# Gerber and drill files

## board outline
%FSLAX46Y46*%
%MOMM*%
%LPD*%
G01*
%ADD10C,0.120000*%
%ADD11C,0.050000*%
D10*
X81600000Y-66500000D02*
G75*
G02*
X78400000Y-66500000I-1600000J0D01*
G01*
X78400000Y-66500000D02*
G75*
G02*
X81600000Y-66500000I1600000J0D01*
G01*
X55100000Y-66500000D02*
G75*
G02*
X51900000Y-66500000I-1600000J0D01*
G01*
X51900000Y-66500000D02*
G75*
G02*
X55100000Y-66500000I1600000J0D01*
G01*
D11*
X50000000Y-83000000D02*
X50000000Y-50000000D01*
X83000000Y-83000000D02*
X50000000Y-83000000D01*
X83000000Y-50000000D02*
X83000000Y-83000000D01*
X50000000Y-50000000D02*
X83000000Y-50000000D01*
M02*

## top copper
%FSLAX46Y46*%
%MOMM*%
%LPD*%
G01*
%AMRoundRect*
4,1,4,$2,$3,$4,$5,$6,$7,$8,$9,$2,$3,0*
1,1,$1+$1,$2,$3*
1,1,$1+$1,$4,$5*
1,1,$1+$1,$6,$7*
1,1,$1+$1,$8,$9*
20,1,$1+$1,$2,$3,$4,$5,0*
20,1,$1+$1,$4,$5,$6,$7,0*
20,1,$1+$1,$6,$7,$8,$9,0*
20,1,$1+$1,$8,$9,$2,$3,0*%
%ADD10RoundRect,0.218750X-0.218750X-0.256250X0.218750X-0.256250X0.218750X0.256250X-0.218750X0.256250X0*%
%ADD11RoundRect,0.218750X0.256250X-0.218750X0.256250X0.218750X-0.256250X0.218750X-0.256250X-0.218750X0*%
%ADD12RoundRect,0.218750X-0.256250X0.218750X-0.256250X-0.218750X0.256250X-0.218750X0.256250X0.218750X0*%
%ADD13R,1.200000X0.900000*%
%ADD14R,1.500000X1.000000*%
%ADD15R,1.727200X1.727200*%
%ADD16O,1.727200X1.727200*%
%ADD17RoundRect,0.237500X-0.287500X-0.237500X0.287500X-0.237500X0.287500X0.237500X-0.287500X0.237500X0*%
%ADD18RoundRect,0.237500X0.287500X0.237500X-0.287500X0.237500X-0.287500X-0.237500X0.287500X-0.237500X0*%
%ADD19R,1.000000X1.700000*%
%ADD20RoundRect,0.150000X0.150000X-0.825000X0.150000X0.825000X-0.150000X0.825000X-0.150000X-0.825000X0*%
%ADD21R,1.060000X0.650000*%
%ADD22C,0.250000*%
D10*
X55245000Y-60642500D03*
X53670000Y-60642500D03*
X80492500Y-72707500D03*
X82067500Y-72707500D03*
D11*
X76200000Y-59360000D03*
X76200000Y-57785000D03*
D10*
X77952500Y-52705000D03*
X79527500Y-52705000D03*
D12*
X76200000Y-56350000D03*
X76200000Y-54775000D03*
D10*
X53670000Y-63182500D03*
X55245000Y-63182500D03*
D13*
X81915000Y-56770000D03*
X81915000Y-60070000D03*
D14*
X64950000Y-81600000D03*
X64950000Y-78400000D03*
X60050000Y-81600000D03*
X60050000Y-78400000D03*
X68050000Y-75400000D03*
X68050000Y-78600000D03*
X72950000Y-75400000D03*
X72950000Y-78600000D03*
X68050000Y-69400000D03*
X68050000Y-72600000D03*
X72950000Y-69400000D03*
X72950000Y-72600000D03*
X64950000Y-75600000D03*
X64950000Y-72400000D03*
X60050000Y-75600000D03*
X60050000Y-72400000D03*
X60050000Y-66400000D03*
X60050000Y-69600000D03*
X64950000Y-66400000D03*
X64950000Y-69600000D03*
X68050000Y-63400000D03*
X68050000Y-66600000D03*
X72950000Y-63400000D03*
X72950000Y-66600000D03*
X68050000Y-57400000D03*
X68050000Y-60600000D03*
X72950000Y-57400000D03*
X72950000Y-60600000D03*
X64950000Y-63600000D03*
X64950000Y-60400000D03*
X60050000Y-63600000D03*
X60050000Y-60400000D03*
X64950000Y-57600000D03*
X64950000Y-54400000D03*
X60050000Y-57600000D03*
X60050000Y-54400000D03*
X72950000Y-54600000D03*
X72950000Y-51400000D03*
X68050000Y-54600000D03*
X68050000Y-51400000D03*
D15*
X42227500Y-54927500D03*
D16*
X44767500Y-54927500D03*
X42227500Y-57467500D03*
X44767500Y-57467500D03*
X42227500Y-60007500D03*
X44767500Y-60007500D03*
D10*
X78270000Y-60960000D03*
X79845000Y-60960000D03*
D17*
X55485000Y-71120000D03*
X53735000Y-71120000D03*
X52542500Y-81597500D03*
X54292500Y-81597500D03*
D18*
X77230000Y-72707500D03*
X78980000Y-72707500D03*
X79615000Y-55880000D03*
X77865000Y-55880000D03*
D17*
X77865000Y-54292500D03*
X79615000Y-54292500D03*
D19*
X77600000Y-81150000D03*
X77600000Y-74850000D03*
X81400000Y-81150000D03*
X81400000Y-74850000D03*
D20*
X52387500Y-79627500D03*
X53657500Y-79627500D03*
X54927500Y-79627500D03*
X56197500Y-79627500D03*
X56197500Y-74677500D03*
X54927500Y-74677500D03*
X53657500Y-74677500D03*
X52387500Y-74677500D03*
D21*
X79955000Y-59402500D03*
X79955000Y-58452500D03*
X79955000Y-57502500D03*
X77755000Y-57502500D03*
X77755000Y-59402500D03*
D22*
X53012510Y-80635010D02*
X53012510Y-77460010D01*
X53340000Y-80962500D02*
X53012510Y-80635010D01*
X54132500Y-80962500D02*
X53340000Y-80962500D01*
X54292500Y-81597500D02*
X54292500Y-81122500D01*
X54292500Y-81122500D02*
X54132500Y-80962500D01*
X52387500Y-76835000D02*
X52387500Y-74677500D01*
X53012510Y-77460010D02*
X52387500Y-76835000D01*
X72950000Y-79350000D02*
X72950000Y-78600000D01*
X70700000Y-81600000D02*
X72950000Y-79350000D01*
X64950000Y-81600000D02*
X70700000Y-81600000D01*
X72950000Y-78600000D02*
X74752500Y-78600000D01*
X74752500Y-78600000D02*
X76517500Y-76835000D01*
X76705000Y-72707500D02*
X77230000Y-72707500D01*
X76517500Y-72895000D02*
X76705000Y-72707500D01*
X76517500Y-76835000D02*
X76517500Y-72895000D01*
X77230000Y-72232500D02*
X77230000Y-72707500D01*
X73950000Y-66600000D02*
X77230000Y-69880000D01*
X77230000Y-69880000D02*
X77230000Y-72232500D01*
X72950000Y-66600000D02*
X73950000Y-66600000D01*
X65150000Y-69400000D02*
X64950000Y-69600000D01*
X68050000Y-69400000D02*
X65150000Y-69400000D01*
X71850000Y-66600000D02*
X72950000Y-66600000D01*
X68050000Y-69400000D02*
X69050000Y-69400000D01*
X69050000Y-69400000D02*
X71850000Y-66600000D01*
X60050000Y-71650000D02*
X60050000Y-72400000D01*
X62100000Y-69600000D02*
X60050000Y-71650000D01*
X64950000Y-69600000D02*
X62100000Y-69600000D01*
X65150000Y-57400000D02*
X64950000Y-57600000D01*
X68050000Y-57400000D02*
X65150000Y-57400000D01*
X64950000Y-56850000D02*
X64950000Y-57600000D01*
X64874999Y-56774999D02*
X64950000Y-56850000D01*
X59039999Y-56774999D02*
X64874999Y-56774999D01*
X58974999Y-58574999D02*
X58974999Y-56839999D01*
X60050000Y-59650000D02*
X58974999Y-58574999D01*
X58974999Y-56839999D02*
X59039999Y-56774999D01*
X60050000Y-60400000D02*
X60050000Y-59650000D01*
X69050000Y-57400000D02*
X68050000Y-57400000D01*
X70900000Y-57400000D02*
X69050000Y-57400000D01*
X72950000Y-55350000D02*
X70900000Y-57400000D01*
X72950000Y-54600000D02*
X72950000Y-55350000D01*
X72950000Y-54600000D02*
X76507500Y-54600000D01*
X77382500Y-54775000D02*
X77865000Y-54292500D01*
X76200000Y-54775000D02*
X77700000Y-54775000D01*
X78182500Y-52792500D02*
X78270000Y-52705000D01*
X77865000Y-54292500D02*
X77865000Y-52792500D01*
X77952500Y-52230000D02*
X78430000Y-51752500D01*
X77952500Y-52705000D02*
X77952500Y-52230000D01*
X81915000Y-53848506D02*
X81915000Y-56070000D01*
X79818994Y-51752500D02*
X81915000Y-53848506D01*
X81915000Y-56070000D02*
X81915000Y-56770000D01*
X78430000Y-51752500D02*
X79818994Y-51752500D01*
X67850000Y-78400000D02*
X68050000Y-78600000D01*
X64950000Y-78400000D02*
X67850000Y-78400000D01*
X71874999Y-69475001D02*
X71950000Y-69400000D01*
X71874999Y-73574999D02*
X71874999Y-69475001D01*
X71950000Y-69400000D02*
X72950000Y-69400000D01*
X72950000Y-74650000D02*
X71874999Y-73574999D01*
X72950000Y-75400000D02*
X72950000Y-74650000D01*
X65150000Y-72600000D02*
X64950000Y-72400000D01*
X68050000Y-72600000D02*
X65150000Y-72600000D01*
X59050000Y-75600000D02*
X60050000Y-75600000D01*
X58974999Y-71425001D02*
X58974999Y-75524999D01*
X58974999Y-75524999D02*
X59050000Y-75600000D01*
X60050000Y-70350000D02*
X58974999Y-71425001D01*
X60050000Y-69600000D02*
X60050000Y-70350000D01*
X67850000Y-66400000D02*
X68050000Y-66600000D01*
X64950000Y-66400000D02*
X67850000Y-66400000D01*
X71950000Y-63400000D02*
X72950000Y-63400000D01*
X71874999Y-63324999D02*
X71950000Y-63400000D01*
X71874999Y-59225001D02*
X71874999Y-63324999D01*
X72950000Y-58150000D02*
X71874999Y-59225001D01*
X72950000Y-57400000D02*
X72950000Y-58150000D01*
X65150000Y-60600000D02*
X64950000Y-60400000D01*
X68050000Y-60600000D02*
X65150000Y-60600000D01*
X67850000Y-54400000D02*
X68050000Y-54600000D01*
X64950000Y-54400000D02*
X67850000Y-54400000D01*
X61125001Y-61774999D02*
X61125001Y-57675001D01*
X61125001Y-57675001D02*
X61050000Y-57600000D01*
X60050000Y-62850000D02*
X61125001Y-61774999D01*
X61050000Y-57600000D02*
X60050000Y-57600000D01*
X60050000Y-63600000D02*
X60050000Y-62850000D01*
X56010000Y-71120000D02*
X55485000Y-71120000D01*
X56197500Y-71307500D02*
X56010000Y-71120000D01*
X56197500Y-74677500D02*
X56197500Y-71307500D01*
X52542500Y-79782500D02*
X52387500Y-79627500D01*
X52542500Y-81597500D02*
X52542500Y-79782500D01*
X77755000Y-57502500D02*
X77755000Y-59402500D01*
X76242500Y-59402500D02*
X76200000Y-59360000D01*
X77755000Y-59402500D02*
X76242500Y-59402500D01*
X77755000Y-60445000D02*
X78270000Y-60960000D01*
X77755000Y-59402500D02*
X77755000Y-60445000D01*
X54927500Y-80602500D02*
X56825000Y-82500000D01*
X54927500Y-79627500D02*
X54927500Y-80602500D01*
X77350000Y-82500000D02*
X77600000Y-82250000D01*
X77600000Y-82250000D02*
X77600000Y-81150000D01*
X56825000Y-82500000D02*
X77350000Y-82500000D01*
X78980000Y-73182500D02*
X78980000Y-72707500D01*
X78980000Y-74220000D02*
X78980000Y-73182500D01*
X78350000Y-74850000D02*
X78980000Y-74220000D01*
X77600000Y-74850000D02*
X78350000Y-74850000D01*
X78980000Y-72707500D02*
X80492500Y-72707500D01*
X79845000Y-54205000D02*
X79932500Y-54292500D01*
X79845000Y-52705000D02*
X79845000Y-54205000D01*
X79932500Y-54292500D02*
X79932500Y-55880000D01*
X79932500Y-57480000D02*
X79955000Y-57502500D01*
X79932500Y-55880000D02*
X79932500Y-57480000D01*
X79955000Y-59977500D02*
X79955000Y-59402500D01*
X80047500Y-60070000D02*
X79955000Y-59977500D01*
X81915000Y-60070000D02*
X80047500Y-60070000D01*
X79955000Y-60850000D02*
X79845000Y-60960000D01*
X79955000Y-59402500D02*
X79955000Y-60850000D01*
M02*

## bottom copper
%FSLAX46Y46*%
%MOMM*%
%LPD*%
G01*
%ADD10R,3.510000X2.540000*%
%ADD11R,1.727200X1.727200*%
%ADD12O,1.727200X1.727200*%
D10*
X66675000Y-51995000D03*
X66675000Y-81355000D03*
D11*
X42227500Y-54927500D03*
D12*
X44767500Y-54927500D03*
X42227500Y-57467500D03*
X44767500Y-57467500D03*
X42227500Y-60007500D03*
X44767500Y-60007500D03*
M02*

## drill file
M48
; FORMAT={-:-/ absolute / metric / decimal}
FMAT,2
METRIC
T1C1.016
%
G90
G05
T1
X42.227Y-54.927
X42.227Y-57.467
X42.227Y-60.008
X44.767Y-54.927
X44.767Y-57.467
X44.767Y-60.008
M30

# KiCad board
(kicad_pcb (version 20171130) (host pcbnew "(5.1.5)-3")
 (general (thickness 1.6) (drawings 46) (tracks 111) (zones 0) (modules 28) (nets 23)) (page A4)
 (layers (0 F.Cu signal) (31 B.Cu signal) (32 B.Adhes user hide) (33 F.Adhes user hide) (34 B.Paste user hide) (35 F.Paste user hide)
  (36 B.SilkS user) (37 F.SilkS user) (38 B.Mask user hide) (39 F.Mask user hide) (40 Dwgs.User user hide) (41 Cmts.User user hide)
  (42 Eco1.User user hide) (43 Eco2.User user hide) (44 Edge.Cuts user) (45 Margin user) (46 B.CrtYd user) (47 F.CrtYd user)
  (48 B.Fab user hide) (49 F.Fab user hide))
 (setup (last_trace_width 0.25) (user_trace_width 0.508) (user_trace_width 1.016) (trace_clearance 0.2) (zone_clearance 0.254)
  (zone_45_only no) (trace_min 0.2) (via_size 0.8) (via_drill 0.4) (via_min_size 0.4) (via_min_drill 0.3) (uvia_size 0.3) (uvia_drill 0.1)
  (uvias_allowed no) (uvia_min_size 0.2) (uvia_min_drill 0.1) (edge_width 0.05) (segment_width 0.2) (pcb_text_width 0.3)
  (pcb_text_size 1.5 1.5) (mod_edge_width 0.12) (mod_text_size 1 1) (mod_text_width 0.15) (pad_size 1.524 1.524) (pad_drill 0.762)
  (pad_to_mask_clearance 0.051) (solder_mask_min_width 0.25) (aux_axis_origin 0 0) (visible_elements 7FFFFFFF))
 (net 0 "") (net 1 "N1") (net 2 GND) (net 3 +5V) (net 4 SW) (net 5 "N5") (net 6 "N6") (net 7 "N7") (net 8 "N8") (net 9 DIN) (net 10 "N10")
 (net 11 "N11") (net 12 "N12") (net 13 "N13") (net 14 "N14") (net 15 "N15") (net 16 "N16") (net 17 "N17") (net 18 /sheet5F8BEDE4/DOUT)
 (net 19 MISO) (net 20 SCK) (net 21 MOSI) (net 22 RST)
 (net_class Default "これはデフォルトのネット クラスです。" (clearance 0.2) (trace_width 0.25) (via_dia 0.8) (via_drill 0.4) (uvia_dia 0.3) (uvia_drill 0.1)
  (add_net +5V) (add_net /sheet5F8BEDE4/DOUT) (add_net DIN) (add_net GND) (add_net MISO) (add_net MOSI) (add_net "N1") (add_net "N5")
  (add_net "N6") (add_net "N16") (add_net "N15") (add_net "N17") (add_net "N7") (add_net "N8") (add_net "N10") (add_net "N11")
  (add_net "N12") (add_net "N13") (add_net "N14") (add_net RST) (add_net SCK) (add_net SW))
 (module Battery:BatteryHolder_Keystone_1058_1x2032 (layer B.Cu) (at 66.675 66.675 270)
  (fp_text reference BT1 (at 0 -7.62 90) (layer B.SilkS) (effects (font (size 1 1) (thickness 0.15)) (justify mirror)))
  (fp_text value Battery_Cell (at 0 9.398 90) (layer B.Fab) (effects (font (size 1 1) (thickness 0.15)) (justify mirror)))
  (pad 1 smd rect (at -14.68 0 270) (size 2.54 3.51) (layers B.Cu B.Paste B.Mask) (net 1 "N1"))
  (pad 2 smd rect (at 14.68 0 270) (size 2.54 3.51) (layers B.Cu B.Paste B.Mask) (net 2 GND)))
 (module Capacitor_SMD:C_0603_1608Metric (layer F.Cu) (at 54.4575 60.6425)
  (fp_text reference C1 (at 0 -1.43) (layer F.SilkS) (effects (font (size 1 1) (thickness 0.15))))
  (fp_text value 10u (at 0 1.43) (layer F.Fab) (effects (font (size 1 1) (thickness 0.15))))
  (pad 2 smd roundrect (at 0.7875 0) (size 0.875 0.95) (layers F.Cu F.Paste F.Mask) (roundrect_rratio 0.25) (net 2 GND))
  (pad 1 smd roundrect (at -0.7875 0) (size 0.875 0.95) (layers F.Cu F.Paste F.Mask) (roundrect_rratio 0.25) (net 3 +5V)))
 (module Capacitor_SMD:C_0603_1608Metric (layer F.Cu) (at 81.28 72.7075)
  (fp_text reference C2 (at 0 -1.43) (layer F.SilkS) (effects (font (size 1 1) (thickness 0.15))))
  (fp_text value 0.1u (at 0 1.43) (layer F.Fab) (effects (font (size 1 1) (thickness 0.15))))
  (pad 1 smd roundrect (at -0.7875 0) (size 0.875 0.95) (layers F.Cu F.Paste F.Mask) (roundrect_rratio 0.25) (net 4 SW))
  (pad 2 smd roundrect (at 0.7875 0) (size 0.875 0.95) (layers F.Cu F.Paste F.Mask) (roundrect_rratio 0.25) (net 2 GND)))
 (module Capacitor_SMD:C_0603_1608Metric (layer F.Cu) (at 76.2 58.5725 90)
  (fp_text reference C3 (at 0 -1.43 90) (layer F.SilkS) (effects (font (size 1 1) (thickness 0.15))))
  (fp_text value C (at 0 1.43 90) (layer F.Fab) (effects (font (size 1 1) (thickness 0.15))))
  (pad 1 smd roundrect (at -0.7875 0 90) (size 0.875 0.95) (layers F.Cu F.Paste F.Mask) (roundrect_rratio 0.25) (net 1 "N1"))
  (pad 2 smd roundrect (at 0.7875 0 90) (size 0.875 0.95) (layers F.Cu F.Paste F.Mask) (roundrect_rratio 0.25) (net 2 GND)))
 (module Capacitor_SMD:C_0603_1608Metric (layer F.Cu) (at 78.74 52.705)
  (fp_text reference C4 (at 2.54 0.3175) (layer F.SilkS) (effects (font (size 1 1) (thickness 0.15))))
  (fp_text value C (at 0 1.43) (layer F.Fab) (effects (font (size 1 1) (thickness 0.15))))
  (pad 1 smd roundrect (at -0.7875 0) (size 0.875 0.95) (layers F.Cu F.Paste F.Mask) (roundrect_rratio 0.25) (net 3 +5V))
  (pad 2 smd roundrect (at 0.7875 0) (size 0.875 0.95) (layers F.Cu F.Paste F.Mask) (roundrect_rratio 0.25) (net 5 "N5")))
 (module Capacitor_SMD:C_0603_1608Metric (layer F.Cu) (at 76.2 55.5625 270)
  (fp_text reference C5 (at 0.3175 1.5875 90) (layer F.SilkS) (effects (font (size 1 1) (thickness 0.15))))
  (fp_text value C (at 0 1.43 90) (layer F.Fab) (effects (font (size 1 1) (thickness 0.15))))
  (pad 2 smd roundrect (at 0.7875 0 270) (size 0.875 0.95) (layers F.Cu F.Paste F.Mask) (roundrect_rratio 0.25) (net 2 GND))
  (pad 1 smd roundrect (at -0.7875 0 270) (size 0.875 0.95) (layers F.Cu F.Paste F.Mask) (roundrect_rratio 0.25) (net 3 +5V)))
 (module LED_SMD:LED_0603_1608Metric (layer F.Cu) (at 54.4575 63.1825)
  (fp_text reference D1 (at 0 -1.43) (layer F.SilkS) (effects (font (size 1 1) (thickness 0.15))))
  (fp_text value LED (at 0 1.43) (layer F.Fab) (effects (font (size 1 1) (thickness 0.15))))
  (pad 1 smd roundrect (at -0.7875 0) (size 0.875 0.95) (layers F.Cu F.Paste F.Mask) (roundrect_rratio 0.25) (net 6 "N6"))
  (pad 2 smd roundrect (at 0.7875 0) (size 0.875 0.95) (layers F.Cu F.Paste F.Mask) (roundrect_rratio 0.25) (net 3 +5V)))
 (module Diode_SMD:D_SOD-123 (layer F.Cu) (at 81.915 58.42 270)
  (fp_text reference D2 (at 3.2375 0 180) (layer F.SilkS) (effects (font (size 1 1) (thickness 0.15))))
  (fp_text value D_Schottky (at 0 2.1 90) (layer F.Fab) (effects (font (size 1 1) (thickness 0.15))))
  (pad 1 smd rect (at -1.65 0 270) (size 0.9 1.2) (layers F.Cu F.Paste F.Mask) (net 3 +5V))
  (pad 2 smd rect (at 1.65 0 270) (size 0.9 1.2) (layers F.Cu F.Paste F.Mask) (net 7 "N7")))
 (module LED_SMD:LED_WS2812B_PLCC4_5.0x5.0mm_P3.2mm (layer F.Cu) (at 62.5 80 180)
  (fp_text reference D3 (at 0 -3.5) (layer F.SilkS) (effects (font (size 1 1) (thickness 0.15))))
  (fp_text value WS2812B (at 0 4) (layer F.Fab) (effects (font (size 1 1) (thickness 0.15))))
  (pad 1 smd rect (at -2.45 -1.6 180) (size 1.5 1) (layers F.Cu F.Paste F.Mask) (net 3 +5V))
  (pad 2 smd rect (at -2.45 1.6 180) (size 1.5 1) (layers F.Cu F.Paste F.Mask) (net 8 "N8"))
  (pad 4 smd rect (at 2.45 -1.6 180) (size 1.5 1) (layers F.Cu F.Paste F.Mask) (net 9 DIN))
  (pad 3 smd rect (at 2.45 1.6 180) (size 1.5 1) (layers F.Cu F.Paste F.Mask) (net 2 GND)))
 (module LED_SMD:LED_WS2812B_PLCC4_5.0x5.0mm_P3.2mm (layer F.Cu) (at 70.5 77 180)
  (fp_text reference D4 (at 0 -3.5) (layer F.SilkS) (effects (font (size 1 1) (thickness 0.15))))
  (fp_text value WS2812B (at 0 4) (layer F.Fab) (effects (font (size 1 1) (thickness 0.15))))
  (pad 3 smd rect (at 2.45 1.6 180) (size 1.5 1) (layers F.Cu F.Paste F.Mask) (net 2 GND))
  (pad 4 smd rect (at 2.45 -1.6 180) (size 1.5 1) (layers F.Cu F.Paste F.Mask) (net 8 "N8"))
  (pad 2 smd rect (at -2.45 1.6 180) (size 1.5 1) (layers F.Cu F.Paste F.Mask) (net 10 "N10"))
  (pad 1 smd rect (at -2.45 -1.6 180) (size 1.5 1) (layers F.Cu F.Paste F.Mask) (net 3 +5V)))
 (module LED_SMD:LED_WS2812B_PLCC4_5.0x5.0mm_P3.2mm (layer F.Cu) (at 70.5 71)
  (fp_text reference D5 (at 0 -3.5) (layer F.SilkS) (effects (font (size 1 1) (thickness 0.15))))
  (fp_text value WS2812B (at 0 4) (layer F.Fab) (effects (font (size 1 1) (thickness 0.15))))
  (pad 1 smd rect (at -2.45 -1.6) (size 1.5 1) (layers F.Cu F.Paste F.Mask) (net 3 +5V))
  (pad 2 smd rect (at -2.45 1.6) (size 1.5 1) (layers F.Cu F.Paste F.Mask) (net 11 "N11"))
  (pad 4 smd rect (at 2.45 -1.6) (size 1.5 1) (layers F.Cu F.Paste F.Mask) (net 10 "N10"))
  (pad 3 smd rect (at 2.45 1.6) (size 1.5 1) (layers F.Cu F.Paste F.Mask) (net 2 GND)))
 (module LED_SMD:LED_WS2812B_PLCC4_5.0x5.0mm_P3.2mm (layer F.Cu) (at 62.5 74)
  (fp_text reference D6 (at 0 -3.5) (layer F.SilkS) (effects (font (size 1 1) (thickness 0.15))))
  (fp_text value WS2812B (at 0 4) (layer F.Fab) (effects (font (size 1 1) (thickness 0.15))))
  (pad 3 smd rect (at 2.45 1.6) (size 1.5 1) (layers F.Cu F.Paste F.Mask) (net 2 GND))
  (pad 4 smd rect (at 2.45 -1.6) (size 1.5 1) (layers F.Cu F.Paste F.Mask) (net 11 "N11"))
  (pad 2 smd rect (at -2.45 1.6) (size 1.5 1) (layers F.Cu F.Paste F.Mask) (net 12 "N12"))
  (pad 1 smd rect (at -2.45 -1.6) (size 1.5 1) (layers F.Cu F.Paste F.Mask) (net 3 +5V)))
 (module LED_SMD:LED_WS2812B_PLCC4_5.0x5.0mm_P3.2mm (layer F.Cu) (at 62.5 68 180)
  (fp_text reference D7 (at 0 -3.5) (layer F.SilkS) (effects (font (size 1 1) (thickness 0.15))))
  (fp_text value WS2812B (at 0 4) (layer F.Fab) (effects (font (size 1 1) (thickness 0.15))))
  (pad 3 smd rect (at 2.45 1.6 180) (size 1.5 1) (layers F.Cu F.Paste F.Mask) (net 2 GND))
  (pad 4 smd rect (at 2.45 -1.6 180) (size 1.5 1) (layers F.Cu F.Paste F.Mask) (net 12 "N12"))
  (pad 2 smd rect (at -2.45 1.6 180) (size 1.5 1) (layers F.Cu F.Paste F.Mask) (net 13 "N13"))
  (pad 1 smd rect (at -2.45 -1.6 180) (size 1.5 1) (layers F.Cu F.Paste F.Mask) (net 3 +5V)))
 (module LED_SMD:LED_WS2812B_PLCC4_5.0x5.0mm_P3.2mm (layer F.Cu) (at 70.5 65 180)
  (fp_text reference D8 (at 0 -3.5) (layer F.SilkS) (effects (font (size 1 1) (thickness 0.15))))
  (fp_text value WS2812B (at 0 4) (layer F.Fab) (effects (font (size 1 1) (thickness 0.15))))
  (pad 3 smd rect (at 2.45 1.6 180) (size 1.5 1) (layers F.Cu F.Paste F.Mask) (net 2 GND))
  (pad 4 smd rect (at 2.45 -1.6 180) (size 1.5 1) (layers F.Cu F.Paste F.Mask) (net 13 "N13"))
  (pad 2 smd rect (at -2.45 1.6 180) (size 1.5 1) (layers F.Cu F.Paste F.Mask) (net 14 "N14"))
  (pad 1 smd rect (at -2.45 -1.6 180) (size 1.5 1) (layers F.Cu F.Paste F.Mask) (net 3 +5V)))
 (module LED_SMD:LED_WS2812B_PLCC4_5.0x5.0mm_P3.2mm (layer F.Cu) (at 70.5 59)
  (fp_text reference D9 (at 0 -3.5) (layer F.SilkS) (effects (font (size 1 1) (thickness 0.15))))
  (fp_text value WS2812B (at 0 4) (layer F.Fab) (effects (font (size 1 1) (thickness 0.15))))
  (pad 1 smd rect (at -2.45 -1.6) (size 1.5 1) (layers F.Cu F.Paste F.Mask) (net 3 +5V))
  (pad 2 smd rect (at -2.45 1.6) (size 1.5 1) (layers F.Cu F.Paste F.Mask) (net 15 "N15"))
  (pad 4 smd rect (at 2.45 -1.6) (size 1.5 1) (layers F.Cu F.Paste F.Mask) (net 14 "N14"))
  (pad 3 smd rect (at 2.45 1.6) (size 1.5 1) (layers F.Cu F.Paste F.Mask) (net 2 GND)))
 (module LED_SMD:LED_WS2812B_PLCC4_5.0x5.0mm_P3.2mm (layer F.Cu) (at 62.5 62)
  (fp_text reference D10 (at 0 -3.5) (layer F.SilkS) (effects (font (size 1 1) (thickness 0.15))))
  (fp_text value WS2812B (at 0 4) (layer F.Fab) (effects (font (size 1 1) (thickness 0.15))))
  (pad 3 smd rect (at 2.45 1.6) (size 1.5 1) (layers F.Cu F.Paste F.Mask) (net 2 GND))
  (pad 4 smd rect (at 2.45 -1.6) (size 1.5 1) (layers F.Cu F.Paste F.Mask) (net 15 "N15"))
  (pad 2 smd rect (at -2.45 1.6) (size 1.5 1) (layers F.Cu F.Paste F.Mask) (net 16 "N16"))
  (pad 1 smd rect (at -2.45 -1.6) (size 1.5 1) (layers F.Cu F.Paste F.Mask) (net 3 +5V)))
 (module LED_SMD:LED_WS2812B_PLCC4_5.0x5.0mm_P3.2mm (layer F.Cu) (at 62.5 56 180)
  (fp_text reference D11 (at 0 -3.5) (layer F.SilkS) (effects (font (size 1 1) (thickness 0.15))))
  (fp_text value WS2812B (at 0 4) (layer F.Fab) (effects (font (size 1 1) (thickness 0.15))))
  (pad 1 smd rect (at -2.45 -1.6 180) (size 1.5 1) (layers F.Cu F.Paste F.Mask) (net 3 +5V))
  (pad 2 smd rect (at -2.45 1.6 180) (size 1.5 1) (layers F.Cu F.Paste F.Mask) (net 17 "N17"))
  (pad 4 smd rect (at 2.45 -1.6 180) (size 1.5 1) (layers F.Cu F.Paste F.Mask) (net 16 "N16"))
  (pad 3 smd rect (at 2.45 1.6 180) (size 1.5 1) (layers F.Cu F.Paste F.Mask) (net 2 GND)))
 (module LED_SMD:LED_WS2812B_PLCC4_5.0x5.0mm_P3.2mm (layer F.Cu) (at 70.5 53 180)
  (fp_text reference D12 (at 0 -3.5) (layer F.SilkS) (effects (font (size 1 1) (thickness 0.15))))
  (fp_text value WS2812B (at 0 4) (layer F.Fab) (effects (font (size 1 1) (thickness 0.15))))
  (pad 1 smd rect (at -2.45 -1.6 180) (size 1.5 1) (layers F.Cu F.Paste F.Mask) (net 3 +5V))
  (pad 2 smd rect (at -2.45 1.6 180) (size 1.5 1) (layers F.Cu F.Paste F.Mask) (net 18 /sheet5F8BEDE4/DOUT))
  (pad 4 smd rect (at 2.45 -1.6 180) (size 1.5 1) (layers F.Cu F.Paste F.Mask) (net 17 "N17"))
  (pad 3 smd rect (at 2.45 1.6 180) (size 1.5 1) (layers F.Cu F.Paste F.Mask) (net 2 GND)))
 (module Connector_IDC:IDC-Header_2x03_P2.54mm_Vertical (layer F.Cu) (at 42.2275 54.9275)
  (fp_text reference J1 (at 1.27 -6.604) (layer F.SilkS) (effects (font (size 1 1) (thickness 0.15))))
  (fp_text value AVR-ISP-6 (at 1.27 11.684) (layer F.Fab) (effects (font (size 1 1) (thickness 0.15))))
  (pad 1 thru_hole rect (at 0 0) (size 1.7272 1.7272) (drill 1.016) (layers *.Cu *.Mask) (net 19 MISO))
  (pad 2 thru_hole oval (at 2.54 0) (size 1.7272 1.7272) (drill 1.016) (layers *.Cu *.Mask) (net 3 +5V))
  (pad 3 thru_hole oval (at 0 2.54) (size 1.7272 1.7272) (drill 1.016) (layers *.Cu *.Mask) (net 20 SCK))
  (pad 4 thru_hole oval (at 2.54 2.54) (size 1.7272 1.7272) (drill 1.016) (layers *.Cu *.Mask) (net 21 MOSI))
  (pad 5 thru_hole oval (at 0 5.08) (size 1.7272 1.7272) (drill 1.016) (layers *.Cu *.Mask) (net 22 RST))
  (pad 6 thru_hole oval (at 2.54 5.08) (size 1.7272 1.7272) (drill 1.016) (layers *.Cu *.Mask) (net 2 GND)))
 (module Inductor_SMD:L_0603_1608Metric (layer F.Cu) (at 79.0575 60.96)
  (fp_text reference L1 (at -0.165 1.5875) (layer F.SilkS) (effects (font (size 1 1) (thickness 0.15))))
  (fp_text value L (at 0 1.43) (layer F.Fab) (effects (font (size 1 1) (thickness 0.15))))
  (pad 1 smd roundrect (at -0.7875 0) (size 0.875 0.95) (layers F.Cu F.Paste F.Mask) (roundrect_rratio 0.25) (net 1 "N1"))
  (pad 2 smd roundrect (at 0.7875 0) (size 0.875 0.95) (layers F.Cu F.Paste F.Mask) (roundrect_rratio 0.25) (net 7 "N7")))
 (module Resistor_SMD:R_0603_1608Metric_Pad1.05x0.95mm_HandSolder (layer F.Cu) (at 54.61 71.12)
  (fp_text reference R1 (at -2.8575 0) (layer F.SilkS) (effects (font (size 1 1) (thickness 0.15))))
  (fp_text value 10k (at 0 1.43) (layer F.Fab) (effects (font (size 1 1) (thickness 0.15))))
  (pad 2 smd roundrect (at 0.875 0) (size 1.05 0.95) (layers F.Cu F.Paste F.Mask) (roundrect_rratio 0.25) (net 21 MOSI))
  (pad 1 smd roundrect (at -0.875 0) (size 1.05 0.95) (layers F.Cu F.Paste F.Mask) (roundrect_rratio 0.25) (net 6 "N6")))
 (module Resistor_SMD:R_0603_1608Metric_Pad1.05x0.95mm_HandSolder (layer F.Cu) (at 53.4175 81.5975)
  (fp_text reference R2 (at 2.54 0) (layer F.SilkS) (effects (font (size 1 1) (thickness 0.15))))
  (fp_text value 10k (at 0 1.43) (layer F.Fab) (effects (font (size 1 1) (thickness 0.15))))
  (pad 1 smd roundrect (at -0.875 0) (size 1.05 0.95) (layers F.Cu F.Paste F.Mask) (roundrect_rratio 0.25) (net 22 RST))
  (pad 2 smd roundrect (at 0.875 0) (size 1.05 0.95) (layers F.Cu F.Paste F.Mask) (roundrect_rratio 0.25) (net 3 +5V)))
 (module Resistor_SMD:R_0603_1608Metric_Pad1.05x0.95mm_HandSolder (layer F.Cu) (at 78.105 72.7075 180)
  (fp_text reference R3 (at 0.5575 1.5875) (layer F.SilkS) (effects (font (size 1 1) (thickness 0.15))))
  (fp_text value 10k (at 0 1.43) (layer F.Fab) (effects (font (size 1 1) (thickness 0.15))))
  (pad 2 smd roundrect (at 0.875 0 180) (size 1.05 0.95) (layers F.Cu F.Paste F.Mask) (roundrect_rratio 0.25) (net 3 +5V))
  (pad 1 smd roundrect (at -0.875 0 180) (size 1.05 0.95) (layers F.Cu F.Paste F.Mask) (roundrect_rratio 0.25) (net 4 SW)))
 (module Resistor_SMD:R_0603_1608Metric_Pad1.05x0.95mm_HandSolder (layer F.Cu) (at 78.74 55.88 180)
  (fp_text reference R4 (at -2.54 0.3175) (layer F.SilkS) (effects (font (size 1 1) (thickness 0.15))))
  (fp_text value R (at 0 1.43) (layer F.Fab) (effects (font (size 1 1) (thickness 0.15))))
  (pad 1 smd roundrect (at -0.875 0 180) (size 1.05 0.95) (layers F.Cu F.Paste F.Mask) (roundrect_rratio 0.25) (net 5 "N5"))
  (pad 2 smd roundrect (at 0.875 0 180) (size 1.05 0.95) (layers F.Cu F.Paste F.Mask) (roundrect_rratio 0.25) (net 2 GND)))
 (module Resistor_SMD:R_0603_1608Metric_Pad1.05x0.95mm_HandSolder (layer F.Cu) (at 78.74 54.2925)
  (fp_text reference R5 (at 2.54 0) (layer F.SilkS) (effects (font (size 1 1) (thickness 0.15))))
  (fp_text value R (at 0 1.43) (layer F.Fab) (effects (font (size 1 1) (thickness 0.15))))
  (pad 1 smd roundrect (at -0.875 0) (size 1.05 0.95) (layers F.Cu F.Paste F.Mask) (roundrect_rratio 0.25) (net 3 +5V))
  (pad 2 smd roundrect (at 0.875 0) (size 1.05 0.95) (layers F.Cu F.Paste F.Mask) (roundrect_rratio 0.25) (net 5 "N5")))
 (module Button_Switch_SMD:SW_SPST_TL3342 (layer F.Cu) (at 79.5 78 90)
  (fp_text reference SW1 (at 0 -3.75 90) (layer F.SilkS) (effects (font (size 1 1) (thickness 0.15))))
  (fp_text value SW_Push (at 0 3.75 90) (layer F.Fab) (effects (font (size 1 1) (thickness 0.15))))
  (pad 1 smd rect (at -3.15 -1.9 90) (size 1.7 1) (layers F.Cu F.Paste F.Mask) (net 4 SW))
  (pad 1 smd rect (at 3.15 -1.9 90) (size 1.7 1) (layers F.Cu F.Paste F.Mask) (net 4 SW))
  (pad 2 smd rect (at -3.15 1.9 90) (size 1.7 1) (layers F.Cu F.Paste F.Mask) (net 2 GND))
  (pad 2 smd rect (at 3.15 1.9 90) (size 1.7 1) (layers F.Cu F.Paste F.Mask) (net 2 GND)))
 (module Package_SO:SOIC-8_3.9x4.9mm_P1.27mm (layer F.Cu) (at 54.2925 77.1525 90)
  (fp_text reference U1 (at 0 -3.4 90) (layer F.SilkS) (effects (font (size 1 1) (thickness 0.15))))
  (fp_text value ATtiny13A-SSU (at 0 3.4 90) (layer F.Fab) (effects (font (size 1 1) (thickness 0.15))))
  (pad 1 smd roundrect (at -2.475 -1.905 90) (size 1.95 0.6) (layers F.Cu F.Paste F.Mask) (roundrect_rratio 0.25) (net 22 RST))
  (pad 2 smd roundrect (at -2.475 -0.635 90) (size 1.95 0.6) (layers F.Cu F.Paste F.Mask) (roundrect_rratio 0.25) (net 9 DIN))
  (pad 3 smd roundrect (at -2.475 0.635 90) (size 1.95 0.6) (layers F.Cu F.Paste F.Mask) (roundrect_rratio 0.25) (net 4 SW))
  (pad 4 smd roundrect (at -2.475 1.905 90) (size 1.95 0.6) (layers F.Cu F.Paste F.Mask) (roundrect_rratio 0.25) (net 2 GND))
  (pad 5 smd roundrect (at 2.475 1.905 90) (size 1.95 0.6) (layers F.Cu F.Paste F.Mask) (roundrect_rratio 0.25) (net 21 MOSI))
  (pad 6 smd roundrect (at 2.475 0.635 90) (size 1.95 0.6) (layers F.Cu F.Paste F.Mask) (roundrect_rratio 0.25) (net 19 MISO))
  (pad 7 smd roundrect (at 2.475 -0.635 90) (size 1.95 0.6) (layers F.Cu F.Paste F.Mask) (roundrect_rratio 0.25) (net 20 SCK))
  (pad 8 smd roundrect (at 2.475 -1.905 90) (size 1.95 0.6) (layers F.Cu F.Paste F.Mask) (roundrect_rratio 0.25) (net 3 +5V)))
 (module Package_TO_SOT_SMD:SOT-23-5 (layer F.Cu) (at 78.855 58.4525 180)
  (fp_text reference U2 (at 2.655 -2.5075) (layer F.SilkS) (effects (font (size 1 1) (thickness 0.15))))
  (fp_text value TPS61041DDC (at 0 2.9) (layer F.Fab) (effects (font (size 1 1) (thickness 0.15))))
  (pad 1 smd rect (at -1.1 -0.95 180) (size 1.06 0.65) (layers F.Cu F.Paste F.Mask) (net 7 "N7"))
  (pad 2 smd rect (at -1.1 0 180) (size 1.06 0.65) (layers F.Cu F.Paste F.Mask) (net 2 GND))
  (pad 3 smd rect (at -1.1 0.95 180) (size 1.06 0.65) (layers F.Cu F.Paste F.Mask) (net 5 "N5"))
  (pad 4 smd rect (at 1.1 0.95 180) (size 1.06 0.65) (layers F.Cu F.Paste F.Mask) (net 1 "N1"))
  (pad 5 smd rect (at 1.1 -0.95 180) (size 1.06 0.65) (layers F.Cu F.Paste F.Mask) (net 1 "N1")))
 (gr_circle (center 80 66.5) (end 81.6 66.5) (layer Edge.Cuts) (width 0.12))
 (gr_circle (center 53.5 66.5) (end 55.1 66.5) (layer Edge.Cuts) (width 0.12))
 (gr_line (start 50 83) (end 50 50) (layer Edge.Cuts) (width 0.05))
 (gr_line (start 83 83) (end 50 83) (layer Edge.Cuts) (width 0.05))
 (gr_line (start 83 50) (end 83 83) (layer Edge.Cuts) (width 0.05))
 (gr_line (start 50 50) (end 83 50) (layer Edge.Cuts) (width 0.05))
 (segment (start 53.01251 80.63501) (end 53.01251 77.46001) (width 0.25) (layer F.Cu) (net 3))
 (segment (start 53.34 80.9625) (end 53.01251 80.63501) (width 0.25) (layer F.Cu) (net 3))
 (segment (start 54.1325 80.9625) (end 53.34 80.9625) (width 0.25) (layer F.Cu) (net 3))
 (segment (start 54.2925 81.5975) (end 54.2925 81.1225) (width 0.25) (layer F.Cu) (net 3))
 (segment (start 54.2925 81.1225) (end 54.1325 80.9625) (width 0.25) (layer F.Cu) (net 3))
 (segment (start 52.3875 76.835) (end 52.3875 74.6775) (width 0.25) (layer F.Cu) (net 3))
 (segment (start 53.01251 77.46001) (end 52.3875 76.835) (width 0.25) (layer F.Cu) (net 3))
 (segment (start 72.95 79.35) (end 72.95 78.6) (width 0.25) (layer F.Cu) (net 3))
 (segment (start 70.7 81.6) (end 72.95 79.35) (width 0.25) (layer F.Cu) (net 3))
 (segment (start 64.95 81.6) (end 70.7 81.6) (width 0.25) (layer F.Cu) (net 3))
 (segment (start 72.95 78.6) (end 74.7525 78.6) (width 0.25) (layer F.Cu) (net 3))
 (segment (start 74.7525 78.6) (end 76.5175 76.835) (width 0.25) (layer F.Cu) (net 3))
 (segment (start 76.705 72.7075) (end 77.23 72.7075) (width 0.25) (layer F.Cu) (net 3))
 (segment (start 76.5175 72.895) (end 76.705 72.7075) (width 0.25) (layer F.Cu) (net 3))
 (segment (start 76.5175 76.835) (end 76.5175 72.895) (width 0.25) (layer F.Cu) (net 3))
 (segment (start 77.23 72.2325) (end 77.23 72.7075) (width 0.25) (layer F.Cu) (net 3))
 (segment (start 73.95 66.6) (end 77.23 69.88) (width 0.25) (layer F.Cu) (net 3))
 (segment (start 77.23 69.88) (end 77.23 72.2325) (width 0.25) (layer F.Cu) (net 3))
 (segment (start 72.95 66.6) (end 73.95 66.6) (width 0.25) (layer F.Cu) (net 3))
 (segment (start 65.15 69.4) (end 64.95 69.6) (width 0.25) (layer F.Cu) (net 3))
 (segment (start 68.05 69.4) (end 65.15 69.4) (width 0.25) (layer F.Cu) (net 3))
 (segment (start 71.85 66.6) (end 72.95 66.6) (width 0.25) (layer F.Cu) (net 3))
 (segment (start 68.05 69.4) (end 69.05 69.4) (width 0.25) (layer F.Cu) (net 3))
 (segment (start 69.05 69.4) (end 71.85 66.6) (width 0.25) (layer F.Cu) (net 3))
 (segment (start 60.05 71.65) (end 60.05 72.4) (width 0.25) (layer F.Cu) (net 3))
 (segment (start 62.1 69.6) (end 60.05 71.65) (width 0.25) (layer F.Cu) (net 3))
 (segment (start 64.95 69.6) (end 62.1 69.6) (width 0.25) (layer F.Cu) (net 3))
 (segment (start 65.15 57.4) (end 64.95 57.6) (width 0.25) (layer F.Cu) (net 3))
 (segment (start 68.05 57.4) (end 65.15 57.4) (width 0.25) (layer F.Cu) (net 3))
 (segment (start 64.95 56.85) (end 64.95 57.6) (width 0.25) (layer F.Cu) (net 3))
 (segment (start 64.874999 56.774999) (end 64.95 56.85) (width 0.25) (layer F.Cu) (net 3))
 (segment (start 59.039999 56.774999) (end 64.874999 56.774999) (width 0.25) (layer F.Cu) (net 3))
 (segment (start 58.974999 58.574999) (end 58.974999 56.839999) (width 0.25) (layer F.Cu) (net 3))
 (segment (start 60.05 59.65) (end 58.974999 58.574999) (width 0.25) (layer F.Cu) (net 3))
 (segment (start 58.974999 56.839999) (end 59.039999 56.774999) (width 0.25) (layer F.Cu) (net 3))
 (segment (start 60.05 60.4) (end 60.05 59.65) (width 0.25) (layer F.Cu) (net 3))
 (segment (start 69.05 57.4) (end 68.05 57.4) (width 0.25) (layer F.Cu) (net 3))
 (segment (start 70.9 57.4) (end 69.05 57.4) (width 0.25) (layer F.Cu) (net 3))
 (segment (start 72.95 55.35) (end 70.9 57.4) (width 0.25) (layer F.Cu) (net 3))
 (segment (start 72.95 54.6) (end 72.95 55.35) (width 0.25) (layer F.Cu) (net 3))
 (segment (start 72.95 54.6) (end 76.5075 54.6) (width 0.25) (layer F.Cu) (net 3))
 (segment (start 77.3825 54.775) (end 77.865 54.2925) (width 0.25) (layer F.Cu) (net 3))
 (segment (start 76.2 54.775) (end 77.7 54.775) (width 0.25) (layer F.Cu) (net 3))
 (segment (start 78.1825 52.7925) (end 78.27 52.705) (width 0.25) (layer F.Cu) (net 3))
 (segment (start 77.865 54.2925) (end 77.865 52.7925) (width 0.25) (layer F.Cu) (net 3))
 (segment (start 77.9525 52.23) (end 78.43 51.7525) (width 0.25) (layer F.Cu) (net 3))
 (segment (start 77.9525 52.705) (end 77.9525 52.23) (width 0.25) (layer F.Cu) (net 3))
 (segment (start 81.915 53.848506) (end 81.915 56.07) (width 0.25) (layer F.Cu) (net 3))
 (segment (start 79.818994 51.7525) (end 81.915 53.848506) (width 0.25) (layer F.Cu) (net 3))
 (segment (start 81.915 56.07) (end 81.915 56.77) (width 0.25) (layer F.Cu) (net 3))
 (segment (start 78.43 51.7525) (end 79.818994 51.7525) (width 0.25) (layer F.Cu) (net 3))
 (segment (start 67.85 78.4) (end 68.05 78.6) (width 0.25) (layer F.Cu) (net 8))
 (segment (start 64.95 78.4) (end 67.85 78.4) (width 0.25) (layer F.Cu) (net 8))
 (segment (start 71.874999 69.475001) (end 71.95 69.4) (width 0.25) (layer F.Cu) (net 10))
 (segment (start 71.874999 73.574999) (end 71.874999 69.475001) (width 0.25) (layer F.Cu) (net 10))
 (segment (start 71.95 69.4) (end 72.95 69.4) (width 0.25) (layer F.Cu) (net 10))
 (segment (start 72.95 74.65) (end 71.874999 73.574999) (width 0.25) (layer F.Cu) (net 10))
 (segment (start 72.95 75.4) (end 72.95 74.65) (width 0.25) (layer F.Cu) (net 10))
 (segment (start 65.15 72.6) (end 64.95 72.4) (width 0.25) (layer F.Cu) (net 11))
 (segment (start 68.05 72.6) (end 65.15 72.6) (width 0.25) (layer F.Cu) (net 11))
 (segment (start 59.05 75.6) (end 60.05 75.6) (width 0.25) (layer F.Cu) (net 12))
 (segment (start 58.974999 71.425001) (end 58.974999 75.524999) (width 0.25) (layer F.Cu) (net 12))
 (segment (start 58.974999 75.524999) (end 59.05 75.6) (width 0.25) (layer F.Cu) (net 12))
 (segment (start 60.05 70.35) (end 58.974999 71.425001) (width 0.25) (layer F.Cu) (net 12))
 (segment (start 60.05 69.6) (end 60.05 70.35) (width 0.25) (layer F.Cu) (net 12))
 (segment (start 67.85 66.4) (end 68.05 66.6) (width 0.25) (layer F.Cu) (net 13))
 (segment (start 64.95 66.4) (end 67.85 66.4) (width 0.25) (layer F.Cu) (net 13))
 (segment (start 71.95 63.4) (end 72.95 63.4) (width 0.25) (layer F.Cu) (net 14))
 (segment (start 71.874999 63.324999) (end 71.95 63.4) (width 0.25) (layer F.Cu) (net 14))
 (segment (start 71.874999 59.225001) (end 71.874999 63.324999) (width 0.25) (layer F.Cu) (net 14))
 (segment (start 72.95 58.15) (end 71.874999 59.225001) (width 0.25) (layer F.Cu) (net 14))
 (segment (start 72.95 57.4) (end 72.95 58.15) (width 0.25) (layer F.Cu) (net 14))
 (segment (start 65.15 60.6) (end 64.95 60.4) (width 0.25) (layer F.Cu) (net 15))
 (segment (start 68.05 60.6) (end 65.15 60.6) (width 0.25) (layer F.Cu) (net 15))
 (segment (start 67.85 54.4) (end 68.05 54.6) (width 0.25) (layer F.Cu) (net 17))
 (segment (start 64.95 54.4) (end 67.85 54.4) (width 0.25) (layer F.Cu) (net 17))
 (segment (start 61.125001 61.774999) (end 61.125001 57.675001) (width 0.25) (layer F.Cu) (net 16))
 (segment (start 61.125001 57.675001) (end 61.05 57.6) (width 0.25) (layer F.Cu) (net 16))
 (segment (start 60.05 62.85) (end 61.125001 61.774999) (width 0.25) (layer F.Cu) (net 16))
 (segment (start 61.05 57.6) (end 60.05 57.6) (width 0.25) (layer F.Cu) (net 16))
 (segment (start 60.05 63.6) (end 60.05 62.85) (width 0.25) (layer F.Cu) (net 16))
 (segment (start 56.01 71.12) (end 55.485 71.12) (width 0.25) (layer F.Cu) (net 21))
 (segment (start 56.1975 71.3075) (end 56.01 71.12) (width 0.25) (layer F.Cu) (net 21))
 (segment (start 56.1975 74.6775) (end 56.1975 71.3075) (width 0.25) (layer F.Cu) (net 21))
 (segment (start 52.5425 79.7825) (end 52.3875 79.6275) (width 0.25) (layer F.Cu) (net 22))
 (segment (start 52.5425 81.5975) (end 52.5425 79.7825) (width 0.25) (layer F.Cu) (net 22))
 (segment (start 77.755 57.5025) (end 77.755 59.4025) (width 0.25) (layer F.Cu) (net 1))
 (segment (start 76.2425 59.4025) (end 76.2 59.36) (width 0.25) (layer F.Cu) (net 1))
 (segment (start 77.755 59.4025) (end 76.2425 59.4025) (width 0.25) (layer F.Cu) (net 1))
 (segment (start 77.755 60.445) (end 78.27 60.96) (width 0.25) (layer F.Cu) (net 1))
 (segment (start 77.755 59.4025) (end 77.755 60.445) (width 0.25) (layer F.Cu) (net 1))
 (segment (start 54.9275 80.6025) (end 56.825 82.5) (width 0.25) (layer F.Cu) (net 4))
 (segment (start 54.9275 79.6275) (end 54.9275 80.6025) (width 0.25) (layer F.Cu) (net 4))
 (segment (start 77.35 82.5) (end 77.6 82.25) (width 0.25) (layer F.Cu) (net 4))
 (segment (start 77.6 82.25) (end 77.6 81.15) (width 0.25) (layer F.Cu) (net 4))
 (segment (start 56.825 82.5) (end 77.35 82.5) (width 0.25) (layer F.Cu) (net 4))
 (segment (start 78.98 73.1825) (end 78.98 72.7075) (width 0.25) (layer F.Cu) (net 4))
 (segment (start 78.98 74.22) (end 78.98 73.1825) (width 0.25) (layer F.Cu) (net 4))
 (segment (start 78.35 74.85) (end 78.98 74.22) (width 0.25) (layer F.Cu) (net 4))
 (segment (start 77.6 74.85) (end 78.35 74.85) (width 0.25) (layer F.Cu) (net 4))
 (segment (start 78.98 72.7075) (end 80.4925 72.7075) (width 0.25) (layer F.Cu) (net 4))
 (segment (start 79.845 54.205) (end 79.9325 54.2925) (width 0.25) (layer F.Cu) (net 5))
 (segment (start 79.845 52.705) (end 79.845 54.205) (width 0.25) (layer F.Cu) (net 5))
 (segment (start 79.9325 54.2925) (end 79.9325 55.88) (width 0.25) (layer F.Cu) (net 5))
 (segment (start 79.9325 57.48) (end 79.955 57.5025) (width 0.25) (layer F.Cu) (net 5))
 (segment (start 79.9325 55.88) (end 79.9325 57.48) (width 0.25) (layer F.Cu) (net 5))
 (segment (start 79.955 59.9775) (end 79.955 59.4025) (width 0.25) (layer F.Cu) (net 7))
 (segment (start 80.0475 60.07) (end 79.955 59.9775) (width 0.25) (layer F.Cu) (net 7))
 (segment (start 81.915 60.07) (end 80.0475 60.07) (width 0.25) (layer F.Cu) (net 7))
 (segment (start 79.955 60.85) (end 79.845 60.96) (width 0.25) (layer F.Cu) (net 7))
 (segment (start 79.955 59.4025) (end 79.955 60.85) (width 0.25) (layer F.Cu) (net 7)))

